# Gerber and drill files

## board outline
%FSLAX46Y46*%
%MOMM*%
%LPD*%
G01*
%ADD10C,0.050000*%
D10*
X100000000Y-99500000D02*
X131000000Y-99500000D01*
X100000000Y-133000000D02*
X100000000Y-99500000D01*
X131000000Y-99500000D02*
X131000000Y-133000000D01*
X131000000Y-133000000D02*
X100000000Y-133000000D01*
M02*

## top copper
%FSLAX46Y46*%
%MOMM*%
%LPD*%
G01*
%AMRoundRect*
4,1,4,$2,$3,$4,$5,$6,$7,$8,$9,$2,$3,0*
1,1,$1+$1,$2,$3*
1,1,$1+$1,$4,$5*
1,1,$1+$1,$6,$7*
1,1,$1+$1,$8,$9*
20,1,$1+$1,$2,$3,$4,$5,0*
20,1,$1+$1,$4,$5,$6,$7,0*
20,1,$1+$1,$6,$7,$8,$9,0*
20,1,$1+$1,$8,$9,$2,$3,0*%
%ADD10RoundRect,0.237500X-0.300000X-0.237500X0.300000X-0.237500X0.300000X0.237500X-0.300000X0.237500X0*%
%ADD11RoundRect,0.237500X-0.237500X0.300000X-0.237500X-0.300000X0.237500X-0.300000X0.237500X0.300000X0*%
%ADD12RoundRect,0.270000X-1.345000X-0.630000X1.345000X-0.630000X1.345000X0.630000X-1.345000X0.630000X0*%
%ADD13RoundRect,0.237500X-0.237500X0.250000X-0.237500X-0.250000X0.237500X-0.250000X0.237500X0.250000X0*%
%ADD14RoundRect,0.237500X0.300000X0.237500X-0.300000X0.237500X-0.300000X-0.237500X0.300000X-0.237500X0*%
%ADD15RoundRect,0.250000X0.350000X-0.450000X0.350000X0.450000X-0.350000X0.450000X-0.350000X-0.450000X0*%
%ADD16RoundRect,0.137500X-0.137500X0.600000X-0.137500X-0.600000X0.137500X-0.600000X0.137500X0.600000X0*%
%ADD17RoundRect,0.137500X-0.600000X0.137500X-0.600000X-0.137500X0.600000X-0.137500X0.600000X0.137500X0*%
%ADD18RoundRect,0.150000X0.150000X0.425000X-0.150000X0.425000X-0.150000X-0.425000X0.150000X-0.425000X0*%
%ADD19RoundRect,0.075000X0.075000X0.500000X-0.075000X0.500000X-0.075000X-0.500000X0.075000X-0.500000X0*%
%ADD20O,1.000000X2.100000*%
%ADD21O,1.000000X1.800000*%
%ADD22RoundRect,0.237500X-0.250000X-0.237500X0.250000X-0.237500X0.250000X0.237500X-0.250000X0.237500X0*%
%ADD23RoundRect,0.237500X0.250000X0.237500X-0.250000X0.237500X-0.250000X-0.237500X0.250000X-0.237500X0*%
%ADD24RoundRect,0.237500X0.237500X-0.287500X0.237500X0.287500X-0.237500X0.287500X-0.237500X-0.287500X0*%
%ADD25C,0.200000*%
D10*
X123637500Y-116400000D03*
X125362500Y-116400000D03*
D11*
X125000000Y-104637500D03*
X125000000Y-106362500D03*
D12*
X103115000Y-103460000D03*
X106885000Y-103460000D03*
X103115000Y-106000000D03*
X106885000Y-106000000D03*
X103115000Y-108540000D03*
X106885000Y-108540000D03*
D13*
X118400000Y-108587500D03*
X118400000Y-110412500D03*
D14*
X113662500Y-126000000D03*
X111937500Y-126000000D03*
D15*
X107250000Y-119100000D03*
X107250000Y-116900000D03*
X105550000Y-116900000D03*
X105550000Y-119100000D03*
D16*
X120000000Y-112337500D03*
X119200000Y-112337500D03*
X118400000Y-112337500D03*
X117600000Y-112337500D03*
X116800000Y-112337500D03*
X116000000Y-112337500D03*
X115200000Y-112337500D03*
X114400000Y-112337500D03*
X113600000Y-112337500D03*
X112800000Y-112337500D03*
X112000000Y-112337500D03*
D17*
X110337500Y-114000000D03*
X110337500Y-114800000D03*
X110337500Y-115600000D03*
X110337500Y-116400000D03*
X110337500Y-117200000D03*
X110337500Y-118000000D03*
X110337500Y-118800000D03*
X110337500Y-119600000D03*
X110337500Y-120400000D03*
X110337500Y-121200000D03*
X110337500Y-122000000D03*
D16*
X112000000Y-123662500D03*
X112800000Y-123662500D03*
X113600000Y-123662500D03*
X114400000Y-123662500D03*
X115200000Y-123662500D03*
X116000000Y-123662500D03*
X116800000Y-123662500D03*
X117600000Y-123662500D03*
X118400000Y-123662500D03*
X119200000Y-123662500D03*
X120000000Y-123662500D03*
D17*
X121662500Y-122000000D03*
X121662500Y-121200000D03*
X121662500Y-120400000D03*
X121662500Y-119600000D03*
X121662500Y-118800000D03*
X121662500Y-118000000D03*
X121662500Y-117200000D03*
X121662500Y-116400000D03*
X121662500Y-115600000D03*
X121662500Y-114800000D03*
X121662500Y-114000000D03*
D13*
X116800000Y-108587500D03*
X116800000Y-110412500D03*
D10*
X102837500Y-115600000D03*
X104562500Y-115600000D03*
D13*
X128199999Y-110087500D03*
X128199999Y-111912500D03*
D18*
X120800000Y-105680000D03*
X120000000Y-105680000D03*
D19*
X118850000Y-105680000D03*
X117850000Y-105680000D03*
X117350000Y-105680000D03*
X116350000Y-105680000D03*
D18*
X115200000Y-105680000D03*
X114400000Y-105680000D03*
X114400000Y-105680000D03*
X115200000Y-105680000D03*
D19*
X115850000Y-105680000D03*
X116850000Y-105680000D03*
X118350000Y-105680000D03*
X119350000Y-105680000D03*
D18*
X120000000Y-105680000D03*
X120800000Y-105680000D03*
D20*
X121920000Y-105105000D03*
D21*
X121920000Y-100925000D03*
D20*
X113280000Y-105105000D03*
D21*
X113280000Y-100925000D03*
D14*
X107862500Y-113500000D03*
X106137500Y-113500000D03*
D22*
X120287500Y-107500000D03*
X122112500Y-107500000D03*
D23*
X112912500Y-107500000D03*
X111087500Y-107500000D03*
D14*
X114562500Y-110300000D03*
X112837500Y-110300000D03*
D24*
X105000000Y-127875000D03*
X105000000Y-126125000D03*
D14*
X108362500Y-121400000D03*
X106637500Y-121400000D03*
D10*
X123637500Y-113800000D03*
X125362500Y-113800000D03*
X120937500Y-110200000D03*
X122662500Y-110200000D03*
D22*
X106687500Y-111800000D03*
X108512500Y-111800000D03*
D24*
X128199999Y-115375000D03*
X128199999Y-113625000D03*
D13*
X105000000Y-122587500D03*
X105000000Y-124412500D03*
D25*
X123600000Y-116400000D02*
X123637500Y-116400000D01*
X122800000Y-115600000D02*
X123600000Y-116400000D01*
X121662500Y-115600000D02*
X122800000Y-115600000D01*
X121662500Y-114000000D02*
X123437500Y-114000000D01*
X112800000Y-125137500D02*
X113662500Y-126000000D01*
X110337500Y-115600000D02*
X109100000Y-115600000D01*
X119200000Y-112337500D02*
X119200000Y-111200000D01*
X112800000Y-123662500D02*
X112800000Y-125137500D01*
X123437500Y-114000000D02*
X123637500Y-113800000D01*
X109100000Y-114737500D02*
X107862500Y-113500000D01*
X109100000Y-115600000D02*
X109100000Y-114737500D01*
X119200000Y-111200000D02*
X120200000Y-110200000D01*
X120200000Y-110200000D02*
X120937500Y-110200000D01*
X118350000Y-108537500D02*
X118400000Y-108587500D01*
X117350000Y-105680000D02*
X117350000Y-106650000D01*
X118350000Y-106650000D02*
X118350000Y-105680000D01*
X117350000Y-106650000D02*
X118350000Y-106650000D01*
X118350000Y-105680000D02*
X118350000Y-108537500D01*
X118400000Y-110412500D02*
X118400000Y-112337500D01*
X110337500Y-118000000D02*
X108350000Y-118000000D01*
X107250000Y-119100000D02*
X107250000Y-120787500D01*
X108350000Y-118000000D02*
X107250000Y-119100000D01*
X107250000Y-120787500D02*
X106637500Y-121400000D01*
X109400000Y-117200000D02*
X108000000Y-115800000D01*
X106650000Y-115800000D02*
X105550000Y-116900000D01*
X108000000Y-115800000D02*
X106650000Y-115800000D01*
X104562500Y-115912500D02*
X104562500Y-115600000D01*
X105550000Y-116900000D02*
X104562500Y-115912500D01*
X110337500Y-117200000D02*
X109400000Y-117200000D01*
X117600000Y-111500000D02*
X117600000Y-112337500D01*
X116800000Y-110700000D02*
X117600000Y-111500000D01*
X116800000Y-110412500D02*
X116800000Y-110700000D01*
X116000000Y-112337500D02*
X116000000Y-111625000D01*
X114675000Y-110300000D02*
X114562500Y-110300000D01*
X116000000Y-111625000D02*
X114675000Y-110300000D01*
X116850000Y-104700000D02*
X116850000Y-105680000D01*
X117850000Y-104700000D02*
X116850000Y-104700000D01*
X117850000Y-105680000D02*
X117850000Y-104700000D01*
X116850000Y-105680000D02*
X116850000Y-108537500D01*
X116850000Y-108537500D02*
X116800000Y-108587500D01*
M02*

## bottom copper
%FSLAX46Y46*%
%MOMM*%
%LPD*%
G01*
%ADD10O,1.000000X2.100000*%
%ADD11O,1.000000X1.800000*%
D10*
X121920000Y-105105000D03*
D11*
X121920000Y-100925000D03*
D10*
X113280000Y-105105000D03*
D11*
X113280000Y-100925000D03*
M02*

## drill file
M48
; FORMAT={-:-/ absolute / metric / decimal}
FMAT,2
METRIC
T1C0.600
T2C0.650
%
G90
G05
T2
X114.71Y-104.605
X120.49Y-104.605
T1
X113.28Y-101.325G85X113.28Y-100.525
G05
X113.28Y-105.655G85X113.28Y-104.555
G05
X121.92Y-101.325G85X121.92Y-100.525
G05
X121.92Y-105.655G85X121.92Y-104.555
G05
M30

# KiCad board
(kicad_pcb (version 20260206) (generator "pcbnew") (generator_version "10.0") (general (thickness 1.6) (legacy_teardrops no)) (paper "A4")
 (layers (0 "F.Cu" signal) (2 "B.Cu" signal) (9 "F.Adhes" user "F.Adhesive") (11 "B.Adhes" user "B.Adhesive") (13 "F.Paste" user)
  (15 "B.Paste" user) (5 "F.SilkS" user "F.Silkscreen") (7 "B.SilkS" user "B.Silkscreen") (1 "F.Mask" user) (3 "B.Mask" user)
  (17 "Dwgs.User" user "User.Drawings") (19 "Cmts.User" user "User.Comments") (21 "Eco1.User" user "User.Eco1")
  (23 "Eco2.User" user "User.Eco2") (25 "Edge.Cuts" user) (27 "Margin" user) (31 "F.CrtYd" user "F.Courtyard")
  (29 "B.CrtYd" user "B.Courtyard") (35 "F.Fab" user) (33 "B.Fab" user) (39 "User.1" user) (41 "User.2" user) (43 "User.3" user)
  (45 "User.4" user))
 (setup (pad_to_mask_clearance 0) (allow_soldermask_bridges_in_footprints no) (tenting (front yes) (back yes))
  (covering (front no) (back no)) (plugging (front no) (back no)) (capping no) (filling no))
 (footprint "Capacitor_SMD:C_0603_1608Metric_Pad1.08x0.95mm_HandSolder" (layer "F.Cu") (at 124.5 116.4)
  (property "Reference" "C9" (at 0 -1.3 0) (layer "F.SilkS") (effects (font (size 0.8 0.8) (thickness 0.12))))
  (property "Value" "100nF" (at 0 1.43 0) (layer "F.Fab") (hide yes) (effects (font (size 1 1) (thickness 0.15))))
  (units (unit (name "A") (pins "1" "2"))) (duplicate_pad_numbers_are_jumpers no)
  (pad "1" smd roundrect (at -0.8625 0) (size 1.075 0.95) (layers "F.Cu" "F.Mask" "F.Paste") (roundrect_rratio 0.25) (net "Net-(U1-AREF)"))
  (pad "2" smd roundrect (at 0.8625 0) (size 1.075 0.95) (layers "F.Cu" "F.Mask" "F.Paste") (roundrect_rratio 0.25) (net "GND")))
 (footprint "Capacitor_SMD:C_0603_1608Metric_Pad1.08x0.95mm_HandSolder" (layer "F.Cu") (at 125 105.5 -90)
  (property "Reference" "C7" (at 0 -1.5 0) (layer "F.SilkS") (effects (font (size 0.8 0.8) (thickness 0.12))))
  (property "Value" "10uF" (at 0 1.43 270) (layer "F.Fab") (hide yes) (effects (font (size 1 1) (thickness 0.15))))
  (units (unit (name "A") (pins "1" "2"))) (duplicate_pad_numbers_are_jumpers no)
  (pad "1" smd roundrect (at -0.8625 0 270) (size 1.075 0.95) (layers "F.Cu" "F.Mask" "F.Paste") (roundrect_rratio 0.25) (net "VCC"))
  (pad "2" smd roundrect (at 0.8625 0 270) (size 1.075 0.95) (layers "F.Cu" "F.Mask" "F.Paste") (roundrect_rratio 0.25) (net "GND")))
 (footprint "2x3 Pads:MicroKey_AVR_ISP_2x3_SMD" (layer "F.Cu") (at 105 106)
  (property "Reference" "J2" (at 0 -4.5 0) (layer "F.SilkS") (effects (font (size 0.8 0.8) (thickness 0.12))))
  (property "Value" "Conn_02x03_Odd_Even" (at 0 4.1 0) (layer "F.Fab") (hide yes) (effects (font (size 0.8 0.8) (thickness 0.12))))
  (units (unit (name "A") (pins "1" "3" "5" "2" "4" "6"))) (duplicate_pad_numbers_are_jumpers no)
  (pad "1" smd roundrect (at -1.885 -2.54) (size 3.23 1.8) (layers "F.Cu" "F.Mask" "F.Paste") (roundrect_rratio 0.15) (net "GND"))
  (pad "2" smd roundrect (at 1.885 -2.54) (size 3.23 1.8) (layers "F.Cu" "F.Mask" "F.Paste") (roundrect_rratio 0.15) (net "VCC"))
  (pad "3" smd roundrect (at -1.885 0) (size 3.23 1.8) (layers "F.Cu" "F.Mask" "F.Paste") (roundrect_rratio 0.15) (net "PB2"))
  (pad "4" smd roundrect (at 1.885 0) (size 3.23 1.8) (layers "F.Cu" "F.Mask" "F.Paste") (roundrect_rratio 0.15) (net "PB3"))
  (pad "5" smd roundrect (at -1.885 2.54) (size 3.23 1.8) (layers "F.Cu" "F.Mask" "F.Paste") (roundrect_rratio 0.15) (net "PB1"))
  (pad "6" smd roundrect (at 1.885 2.54) (size 3.23 1.8) (layers "F.Cu" "F.Mask" "F.Paste") (roundrect_rratio 0.15) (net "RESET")))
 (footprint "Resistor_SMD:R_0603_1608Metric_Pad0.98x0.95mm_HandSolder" (layer "F.Cu") (at 118.4 109.5 -90)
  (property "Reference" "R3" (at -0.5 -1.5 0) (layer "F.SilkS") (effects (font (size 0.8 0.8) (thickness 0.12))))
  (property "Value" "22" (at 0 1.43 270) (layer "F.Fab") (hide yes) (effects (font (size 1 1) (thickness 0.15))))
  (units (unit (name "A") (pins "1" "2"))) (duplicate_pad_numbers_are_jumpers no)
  (pad "1" smd roundrect (at -0.9125 0 270) (size 0.975 0.95) (layers "F.Cu" "F.Mask" "F.Paste") (roundrect_rratio 0.25)
   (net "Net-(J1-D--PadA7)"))
  (pad "2" smd roundrect (at 0.9125 0 270) (size 0.975 0.95) (layers "F.Cu" "F.Mask" "F.Paste") (roundrect_rratio 0.25) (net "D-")))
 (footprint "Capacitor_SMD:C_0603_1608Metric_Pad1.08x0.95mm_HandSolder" (layer "F.Cu") (at 112.8 126 180)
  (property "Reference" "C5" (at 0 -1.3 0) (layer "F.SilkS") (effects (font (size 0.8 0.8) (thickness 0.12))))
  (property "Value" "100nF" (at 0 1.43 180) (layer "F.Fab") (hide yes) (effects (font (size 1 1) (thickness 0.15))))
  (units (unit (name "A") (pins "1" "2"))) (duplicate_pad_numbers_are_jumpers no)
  (pad "1" smd roundrect (at -0.8625 0 180) (size 1.075 0.95) (layers "F.Cu" "F.Mask" "F.Paste") (roundrect_rratio 0.25) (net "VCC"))
  (pad "2" smd roundrect (at 0.8625 0 180) (size 1.075 0.95) (layers "F.Cu" "F.Mask" "F.Paste") (roundrect_rratio 0.25) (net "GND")))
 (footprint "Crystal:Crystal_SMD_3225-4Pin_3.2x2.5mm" (layer "F.Cu") (at 106.4 118 90)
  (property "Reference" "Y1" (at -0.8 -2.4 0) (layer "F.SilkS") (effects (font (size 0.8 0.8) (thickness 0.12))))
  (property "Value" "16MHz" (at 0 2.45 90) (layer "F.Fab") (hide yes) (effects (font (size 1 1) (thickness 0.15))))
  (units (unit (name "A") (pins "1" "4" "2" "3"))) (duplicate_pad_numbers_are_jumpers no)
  (pad "1" smd roundrect (at -1.1 0.85 90) (size 1.4 1.2) (layers "F.Cu" "F.Mask" "F.Paste") (roundrect_rratio 0.208333)
   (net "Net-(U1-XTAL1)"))
  (pad "2" smd roundrect (at 1.1 0.85 90) (size 1.4 1.2) (layers "F.Cu" "F.Mask" "F.Paste") (roundrect_rratio 0.208333) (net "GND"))
  (pad "3" smd roundrect (at 1.1 -0.85 90) (size 1.4 1.2) (layers "F.Cu" "F.Mask" "F.Paste") (roundrect_rratio 0.208333)
   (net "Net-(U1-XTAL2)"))
  (pad "4" smd roundrect (at -1.1 -0.85 90) (size 1.4 1.2) (layers "F.Cu" "F.Mask" "F.Paste") (roundrect_rratio 0.208333) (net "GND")))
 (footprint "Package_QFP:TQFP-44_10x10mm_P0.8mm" (layer "F.Cu") (at 116 118 -90)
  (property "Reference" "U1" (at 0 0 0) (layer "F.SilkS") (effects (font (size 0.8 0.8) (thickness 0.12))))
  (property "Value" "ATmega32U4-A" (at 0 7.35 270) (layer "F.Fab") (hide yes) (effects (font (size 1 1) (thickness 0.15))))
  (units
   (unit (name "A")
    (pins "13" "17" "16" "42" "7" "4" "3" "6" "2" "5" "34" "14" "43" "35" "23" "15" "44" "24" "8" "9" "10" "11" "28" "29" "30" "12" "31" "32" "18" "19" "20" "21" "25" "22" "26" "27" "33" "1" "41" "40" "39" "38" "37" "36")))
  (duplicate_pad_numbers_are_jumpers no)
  (pad "1" smd roundrect (at -5.6625 -4 270) (size 1.475 0.55) (layers "F.Cu" "F.Mask" "F.Paste") (roundrect_rratio 0.25)
   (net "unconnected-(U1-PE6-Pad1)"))
  (pad "2" smd roundrect (at -5.6625 -3.2 270) (size 1.475 0.55) (layers "F.Cu" "F.Mask" "F.Paste") (roundrect_rratio 0.25) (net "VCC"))
  (pad "3" smd roundrect (at -5.6625 -2.4 270) (size 1.475 0.55) (layers "F.Cu" "F.Mask" "F.Paste") (roundrect_rratio 0.25) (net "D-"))
  (pad "4" smd roundrect (at -5.6625 -1.6 270) (size 1.475 0.55) (layers "F.Cu" "F.Mask" "F.Paste") (roundrect_rratio 0.25) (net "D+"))
  (pad "5" smd roundrect (at -5.6625 -0.8 270) (size 1.475 0.55) (layers "F.Cu" "F.Mask" "F.Paste") (roundrect_rratio 0.25) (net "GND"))
  (pad "6" smd roundrect (at -5.6625 0 270) (size 1.475 0.55) (layers "F.Cu" "F.Mask" "F.Paste") (roundrect_rratio 0.25)
   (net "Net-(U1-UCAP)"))
  (pad "7" smd roundrect (at -5.6625 0.8 270) (size 1.475 0.55) (layers "F.Cu" "F.Mask" "F.Paste") (roundrect_rratio 0.25) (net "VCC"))
  (pad "8" smd roundrect (at -5.6625 1.6 270) (size 1.475 0.55) (layers "F.Cu" "F.Mask" "F.Paste") (roundrect_rratio 0.25)
   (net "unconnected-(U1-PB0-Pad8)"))
  (pad "9" smd roundrect (at -5.6625 2.4 270) (size 1.475 0.55) (layers "F.Cu" "F.Mask" "F.Paste") (roundrect_rratio 0.25) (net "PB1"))
  (pad "10" smd roundrect (at -5.6625 3.2 270) (size 1.475 0.55) (layers "F.Cu" "F.Mask" "F.Paste") (roundrect_rratio 0.25) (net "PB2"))
  (pad "11" smd roundrect (at -5.6625 4 270) (size 1.475 0.55) (layers "F.Cu" "F.Mask" "F.Paste") (roundrect_rratio 0.25) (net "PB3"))
  (pad "12" smd roundrect (at -4 5.6625 270) (size 0.55 1.475) (layers "F.Cu" "F.Mask" "F.Paste") (roundrect_rratio 0.25)
   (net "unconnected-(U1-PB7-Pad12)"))
  (pad "13" smd roundrect (at -3.2 5.6625 270) (size 0.55 1.475) (layers "F.Cu" "F.Mask" "F.Paste") (roundrect_rratio 0.25) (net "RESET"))
  (pad "14" smd roundrect (at -2.4 5.6625 270) (size 0.55 1.475) (layers "F.Cu" "F.Mask" "F.Paste") (roundrect_rratio 0.25) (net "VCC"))
  (pad "15" smd roundrect (at -1.6 5.6625 270) (size 0.55 1.475) (layers "F.Cu" "F.Mask" "F.Paste") (roundrect_rratio 0.25) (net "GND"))
  (pad "16" smd roundrect (at -0.8 5.6625 270) (size 0.55 1.475) (layers "F.Cu" "F.Mask" "F.Paste") (roundrect_rratio 0.25)
   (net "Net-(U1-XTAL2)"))
  (pad "17" smd roundrect (at 0 5.6625 270) (size 0.55 1.475) (layers "F.Cu" "F.Mask" "F.Paste") (roundrect_rratio 0.25)
   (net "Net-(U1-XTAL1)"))
  (pad "18" smd roundrect (at 0.8 5.6625 270) (size 0.55 1.475) (layers "F.Cu" "F.Mask" "F.Paste") (roundrect_rratio 0.25)
   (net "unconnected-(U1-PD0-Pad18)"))
  (pad "19" smd roundrect (at 1.6 5.6625 270) (size 0.55 1.475) (layers "F.Cu" "F.Mask" "F.Paste") (roundrect_rratio 0.25)
   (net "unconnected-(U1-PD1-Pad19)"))
  (pad "20" smd roundrect (at 2.4 5.6625 270) (size 0.55 1.475) (layers "F.Cu" "F.Mask" "F.Paste") (roundrect_rratio 0.25)
   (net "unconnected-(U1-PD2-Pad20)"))
  (pad "21" smd roundrect (at 3.2 5.6625 270) (size 0.55 1.475) (layers "F.Cu" "F.Mask" "F.Paste") (roundrect_rratio 0.25)
   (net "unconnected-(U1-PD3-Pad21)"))
  (pad "22" smd roundrect (at 4 5.6625 270) (size 0.55 1.475) (layers "F.Cu" "F.Mask" "F.Paste") (roundrect_rratio 0.25)
   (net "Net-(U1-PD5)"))
  (pad "23" smd roundrect (at 5.6625 4 270) (size 1.475 0.55) (layers "F.Cu" "F.Mask" "F.Paste") (roundrect_rratio 0.25) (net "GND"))
  (pad "24" smd roundrect (at 5.6625 3.2 270) (size 1.475 0.55) (layers "F.Cu" "F.Mask" "F.Paste") (roundrect_rratio 0.25) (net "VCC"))
  (pad "25" smd roundrect (at 5.6625 2.4 270) (size 1.475 0.55) (layers "F.Cu" "F.Mask" "F.Paste") (roundrect_rratio 0.25)
   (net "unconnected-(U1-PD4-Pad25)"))
  (pad "26" smd roundrect (at 5.6625 1.6 270) (size 1.475 0.55) (layers "F.Cu" "F.Mask" "F.Paste") (roundrect_rratio 0.25)
   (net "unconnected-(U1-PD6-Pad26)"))
  (pad "27" smd roundrect (at 5.6625 0.8 270) (size 1.475 0.55) (layers "F.Cu" "F.Mask" "F.Paste") (roundrect_rratio 0.25)
   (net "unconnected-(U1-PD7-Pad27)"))
  (pad "28" smd roundrect (at 5.6625 0 270) (size 1.475 0.55) (layers "F.Cu" "F.Mask" "F.Paste") (roundrect_rratio 0.25)
   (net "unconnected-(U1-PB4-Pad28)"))
  (pad "29" smd roundrect (at 5.6625 -0.8 270) (size 1.475 0.55) (layers "F.Cu" "F.Mask" "F.Paste") (roundrect_rratio 0.25)
   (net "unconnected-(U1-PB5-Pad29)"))
  (pad "30" smd roundrect (at 5.6625 -1.6 270) (size 1.475 0.55) (layers "F.Cu" "F.Mask" "F.Paste") (roundrect_rratio 0.25)
   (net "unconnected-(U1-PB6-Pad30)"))
  (pad "31" smd roundrect (at 5.6625 -2.4 270) (size 1.475 0.55) (layers "F.Cu" "F.Mask" "F.Paste") (roundrect_rratio 0.25)
   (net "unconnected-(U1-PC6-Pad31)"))
  (pad "32" smd roundrect (at 5.6625 -3.2 270) (size 1.475 0.55) (layers "F.Cu" "F.Mask" "F.Paste") (roundrect_rratio 0.25)
   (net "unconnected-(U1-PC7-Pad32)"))
  (pad "33" smd roundrect (at 5.6625 -4 270) (size 1.475 0.55) (layers "F.Cu" "F.Mask" "F.Paste") (roundrect_rratio 0.25)
   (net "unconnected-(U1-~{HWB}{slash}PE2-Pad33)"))
  (pad "34" smd roundrect (at 4 -5.6625 270) (size 0.55 1.475) (layers "F.Cu" "F.Mask" "F.Paste") (roundrect_rratio 0.25) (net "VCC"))
  (pad "35" smd roundrect (at 3.2 -5.6625 270) (size 0.55 1.475) (layers "F.Cu" "F.Mask" "F.Paste") (roundrect_rratio 0.25) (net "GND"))
  (pad "36" smd roundrect (at 2.4 -5.6625 270) (size 0.55 1.475) (layers "F.Cu" "F.Mask" "F.Paste") (roundrect_rratio 0.25)
   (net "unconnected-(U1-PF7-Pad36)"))
  (pad "37" smd roundrect (at 1.6 -5.6625 270) (size 0.55 1.475) (layers "F.Cu" "F.Mask" "F.Paste") (roundrect_rratio 0.25)
   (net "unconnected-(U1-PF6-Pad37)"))
  (pad "38" smd roundrect (at 0.8 -5.6625 270) (size 0.55 1.475) (layers "F.Cu" "F.Mask" "F.Paste") (roundrect_rratio 0.25)
   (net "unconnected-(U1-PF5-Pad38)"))
  (pad "39" smd roundrect (at 0 -5.6625 270) (size 0.55 1.475) (layers "F.Cu" "F.Mask" "F.Paste") (roundrect_rratio 0.25)
   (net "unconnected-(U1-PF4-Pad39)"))
  (pad "40" smd roundrect (at -0.8 -5.6625 270) (size 0.55 1.475) (layers "F.Cu" "F.Mask" "F.Paste") (roundrect_rratio 0.25)
   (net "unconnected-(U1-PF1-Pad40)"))
  (pad "41" smd roundrect (at -1.6 -5.6625 270) (size 0.55 1.475) (layers "F.Cu" "F.Mask" "F.Paste") (roundrect_rratio 0.25)
   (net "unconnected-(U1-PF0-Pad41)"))
  (pad "42" smd roundrect (at -2.4 -5.6625 270) (size 0.55 1.475) (layers "F.Cu" "F.Mask" "F.Paste") (roundrect_rratio 0.25)
   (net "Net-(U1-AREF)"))
  (pad "43" smd roundrect (at -3.2 -5.6625 270) (size 0.55 1.475) (layers "F.Cu" "F.Mask" "F.Paste") (roundrect_rratio 0.25) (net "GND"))
  (pad "44" smd roundrect (at -4 -5.6625 270) (size 0.55 1.475) (layers "F.Cu" "F.Mask" "F.Paste") (roundrect_rratio 0.25) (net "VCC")))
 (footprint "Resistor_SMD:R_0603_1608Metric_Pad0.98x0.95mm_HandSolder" (layer "F.Cu") (at 116.8 109.5 -90)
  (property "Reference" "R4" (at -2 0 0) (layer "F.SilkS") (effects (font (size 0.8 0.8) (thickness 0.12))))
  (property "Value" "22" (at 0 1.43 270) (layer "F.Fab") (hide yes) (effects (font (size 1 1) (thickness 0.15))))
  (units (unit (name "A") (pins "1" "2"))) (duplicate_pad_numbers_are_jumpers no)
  (pad "1" smd roundrect (at -0.9125 0 270) (size 0.975 0.95) (layers "F.Cu" "F.Mask" "F.Paste") (roundrect_rratio 0.25)
   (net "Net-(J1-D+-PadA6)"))
  (pad "2" smd roundrect (at 0.9125 0 270) (size 0.975 0.95) (layers "F.Cu" "F.Mask" "F.Paste") (roundrect_rratio 0.25) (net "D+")))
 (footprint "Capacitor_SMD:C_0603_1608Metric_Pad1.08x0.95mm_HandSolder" (layer "F.Cu") (at 103.7 115.6)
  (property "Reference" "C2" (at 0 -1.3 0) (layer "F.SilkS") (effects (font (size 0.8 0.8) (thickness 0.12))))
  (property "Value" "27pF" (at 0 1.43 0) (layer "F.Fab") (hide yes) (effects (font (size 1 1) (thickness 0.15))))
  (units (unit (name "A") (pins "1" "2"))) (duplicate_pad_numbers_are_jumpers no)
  (pad "1" smd roundrect (at -0.8625 0) (size 1.075 0.95) (layers "F.Cu" "F.Mask" "F.Paste") (roundrect_rratio 0.25) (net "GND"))
  (pad "2" smd roundrect (at 0.8625 0) (size 1.075 0.95) (layers "F.Cu" "F.Mask" "F.Paste") (roundrect_rratio 0.25) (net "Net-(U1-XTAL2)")))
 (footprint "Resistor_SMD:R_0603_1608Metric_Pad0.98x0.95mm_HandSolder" (layer "F.Cu") (at 128.199999 111 -90)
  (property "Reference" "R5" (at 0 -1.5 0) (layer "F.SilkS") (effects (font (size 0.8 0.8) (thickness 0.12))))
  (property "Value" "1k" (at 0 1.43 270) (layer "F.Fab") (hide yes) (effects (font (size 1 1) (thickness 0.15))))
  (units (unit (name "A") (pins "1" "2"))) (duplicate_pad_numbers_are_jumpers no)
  (pad "1" smd roundrect (at -0.9125 0 270) (size 0.975 0.95) (layers "F.Cu" "F.Mask" "F.Paste") (roundrect_rratio 0.25) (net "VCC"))
  (pad "2" smd roundrect (at 0.9125 0 270) (size 0.975 0.95) (layers "F.Cu" "F.Mask" "F.Paste") (roundrect_rratio 0.25) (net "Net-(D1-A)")))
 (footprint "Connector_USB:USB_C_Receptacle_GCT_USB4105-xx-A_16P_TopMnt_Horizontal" (layer "F.Cu") (at 117.6 102 180)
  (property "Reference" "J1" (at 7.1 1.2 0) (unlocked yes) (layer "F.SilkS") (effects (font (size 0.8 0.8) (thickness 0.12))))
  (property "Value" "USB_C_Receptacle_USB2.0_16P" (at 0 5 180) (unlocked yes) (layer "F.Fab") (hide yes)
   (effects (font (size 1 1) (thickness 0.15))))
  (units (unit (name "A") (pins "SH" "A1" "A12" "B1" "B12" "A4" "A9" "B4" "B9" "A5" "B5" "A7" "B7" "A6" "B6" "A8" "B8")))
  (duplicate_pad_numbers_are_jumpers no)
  (pad "" np_thru_hole circle (at -2.89 -2.605 180) (size 0.65 0.65) (drill 0.65) (layers "*.Cu" "*.Mask"))
  (pad "" np_thru_hole circle (at 2.89 -2.605 180) (size 0.65 0.65) (drill 0.65) (layers "*.Cu" "*.Mask"))
  (pad "A1" smd roundrect (at -3.2 -3.68 180) (size 0.6 1.15) (layers "F.Cu" "F.Mask" "F.Paste") (roundrect_rratio 0.25) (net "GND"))
  (pad "A4" smd roundrect (at -2.4 -3.68 180) (size 0.6 1.15) (layers "F.Cu" "F.Mask" "F.Paste") (roundrect_rratio 0.25) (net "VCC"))
  (pad "A5" smd roundrect (at -1.25 -3.68 180) (size 0.3 1.15) (layers "F.Cu" "F.Mask" "F.Paste") (roundrect_rratio 0.25)
   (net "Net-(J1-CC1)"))
  (pad "A6" smd roundrect (at -0.25 -3.68 180) (size 0.3 1.15) (layers "F.Cu" "F.Mask" "F.Paste") (roundrect_rratio 0.25)
   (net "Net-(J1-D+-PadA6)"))
  (pad "A7" smd roundrect (at 0.25 -3.68 180) (size 0.3 1.15) (layers "F.Cu" "F.Mask" "F.Paste") (roundrect_rratio 0.25)
   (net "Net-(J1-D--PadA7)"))
  (pad "A8" smd roundrect (at 1.25 -3.68 180) (size 0.3 1.15) (layers "F.Cu" "F.Mask" "F.Paste") (roundrect_rratio 0.25)
   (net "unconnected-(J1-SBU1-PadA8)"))
  (pad "A9" smd roundrect (at 2.4 -3.68 180) (size 0.6 1.15) (layers "F.Cu" "F.Mask" "F.Paste") (roundrect_rratio 0.25) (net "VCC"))
  (pad "A12" smd roundrect (at 3.2 -3.68 180) (size 0.6 1.15) (layers "F.Cu" "F.Mask" "F.Paste") (roundrect_rratio 0.25) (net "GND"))
  (pad "B1" smd roundrect (at 3.2 -3.68 180) (size 0.6 1.15) (layers "F.Cu" "F.Mask" "F.Paste") (roundrect_rratio 0.25) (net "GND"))
  (pad "B4" smd roundrect (at 2.4 -3.68 180) (size 0.6 1.15) (layers "F.Cu" "F.Mask" "F.Paste") (roundrect_rratio 0.25) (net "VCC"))
  (pad "B5" smd roundrect (at 1.75 -3.68 180) (size 0.3 1.15) (layers "F.Cu" "F.Mask" "F.Paste") (roundrect_rratio 0.25)
   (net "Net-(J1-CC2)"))
  (pad "B6" smd roundrect (at 0.75 -3.68 180) (size 0.3 1.15) (layers "F.Cu" "F.Mask" "F.Paste") (roundrect_rratio 0.25)
   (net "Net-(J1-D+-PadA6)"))
  (pad "B7" smd roundrect (at -0.75 -3.68 180) (size 0.3 1.15) (layers "F.Cu" "F.Mask" "F.Paste") (roundrect_rratio 0.25)
   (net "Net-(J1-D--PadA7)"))
  (pad "B8" smd roundrect (at -1.75 -3.68 180) (size 0.3 1.15) (layers "F.Cu" "F.Mask" "F.Paste") (roundrect_rratio 0.25)
   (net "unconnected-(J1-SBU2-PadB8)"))
  (pad "B9" smd roundrect (at -2.4 -3.68 180) (size 0.6 1.15) (layers "F.Cu" "F.Mask" "F.Paste") (roundrect_rratio 0.25) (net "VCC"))
  (pad "B12" smd roundrect (at -3.2 -3.68 180) (size 0.6 1.15) (layers "F.Cu" "F.Mask" "F.Paste") (roundrect_rratio 0.25) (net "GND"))
  (pad "SH" thru_hole oval (at -4.32 -3.105 180) (size 1 2.1) (drill oval 0.6 1.7) (layers "*.Cu" "*.Mask" "F.Paste")
   (remove_unused_layers no) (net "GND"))
  (pad "SH" thru_hole oval (at -4.32 1.075 180) (size 1 1.8) (drill oval 0.6 1.4) (layers "*.Cu" "*.Mask" "F.Paste")
   (remove_unused_layers no) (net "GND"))
  (pad "SH" thru_hole oval (at 4.32 -3.105 180) (size 1 2.1) (drill oval 0.6 1.7) (layers "*.Cu" "*.Mask" "F.Paste")
   (remove_unused_layers no) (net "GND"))
  (pad "SH" thru_hole oval (at 4.32 1.075 180) (size 1 1.8) (drill oval 0.6 1.4) (layers "*.Cu" "*.Mask" "F.Paste")
   (remove_unused_layers no) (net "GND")))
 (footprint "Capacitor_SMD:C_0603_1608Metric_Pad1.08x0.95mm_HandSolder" (layer "F.Cu") (at 107 113.5 180)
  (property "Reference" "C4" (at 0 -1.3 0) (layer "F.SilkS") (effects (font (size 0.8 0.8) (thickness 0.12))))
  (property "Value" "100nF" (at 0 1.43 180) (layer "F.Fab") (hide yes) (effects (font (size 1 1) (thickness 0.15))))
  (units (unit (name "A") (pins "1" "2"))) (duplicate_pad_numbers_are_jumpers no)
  (pad "1" smd roundrect (at -0.8625 0 180) (size 1.075 0.95) (layers "F.Cu" "F.Mask" "F.Paste") (roundrect_rratio 0.25) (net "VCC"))
  (pad "2" smd roundrect (at 0.8625 0 180) (size 1.075 0.95) (layers "F.Cu" "F.Mask" "F.Paste") (roundrect_rratio 0.25) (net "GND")))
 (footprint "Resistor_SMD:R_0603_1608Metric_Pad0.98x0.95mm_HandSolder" (layer "F.Cu") (at 121.2 107.5)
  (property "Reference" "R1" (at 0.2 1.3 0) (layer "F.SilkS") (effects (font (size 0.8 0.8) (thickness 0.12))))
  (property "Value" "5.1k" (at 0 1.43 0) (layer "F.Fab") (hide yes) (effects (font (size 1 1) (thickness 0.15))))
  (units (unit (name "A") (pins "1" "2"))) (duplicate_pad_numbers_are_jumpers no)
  (pad "1" smd roundrect (at -0.9125 0) (size 0.975 0.95) (layers "F.Cu" "F.Mask" "F.Paste") (roundrect_rratio 0.25) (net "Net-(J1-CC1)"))
  (pad "2" smd roundrect (at 0.9125 0) (size 0.975 0.95) (layers "F.Cu" "F.Mask" "F.Paste") (roundrect_rratio 0.25) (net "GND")))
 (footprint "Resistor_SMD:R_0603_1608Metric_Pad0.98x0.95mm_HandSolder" (layer "F.Cu") (at 112 107.5 180)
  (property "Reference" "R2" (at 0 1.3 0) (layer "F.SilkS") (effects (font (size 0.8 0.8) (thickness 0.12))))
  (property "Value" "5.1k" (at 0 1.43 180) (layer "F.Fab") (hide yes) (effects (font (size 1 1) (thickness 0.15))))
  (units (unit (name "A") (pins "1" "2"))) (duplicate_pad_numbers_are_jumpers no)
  (pad "1" smd roundrect (at -0.9125 0 180) (size 0.975 0.95) (layers "F.Cu" "F.Mask" "F.Paste") (roundrect_rratio 0.25)
   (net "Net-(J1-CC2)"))
  (pad "2" smd roundrect (at 0.9125 0 180) (size 0.975 0.95) (layers "F.Cu" "F.Mask" "F.Paste") (roundrect_rratio 0.25) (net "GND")))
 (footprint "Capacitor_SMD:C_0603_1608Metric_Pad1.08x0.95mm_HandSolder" (layer "F.Cu") (at 113.7 110.3 180)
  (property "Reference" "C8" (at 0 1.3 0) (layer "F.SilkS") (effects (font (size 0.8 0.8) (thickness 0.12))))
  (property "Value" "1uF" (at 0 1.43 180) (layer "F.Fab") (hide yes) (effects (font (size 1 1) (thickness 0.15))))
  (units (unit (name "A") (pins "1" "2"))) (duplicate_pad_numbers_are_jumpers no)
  (pad "1" smd roundrect (at -0.8625 0 180) (size 1.075 0.95) (layers "F.Cu" "F.Mask" "F.Paste") (roundrect_rratio 0.25)
   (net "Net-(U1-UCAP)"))
  (pad "2" smd roundrect (at 0.8625 0 180) (size 1.075 0.95) (layers "F.Cu" "F.Mask" "F.Paste") (roundrect_rratio 0.25) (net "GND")))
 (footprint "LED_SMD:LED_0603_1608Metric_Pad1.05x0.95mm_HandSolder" (layer "F.Cu") (at 105 127 90)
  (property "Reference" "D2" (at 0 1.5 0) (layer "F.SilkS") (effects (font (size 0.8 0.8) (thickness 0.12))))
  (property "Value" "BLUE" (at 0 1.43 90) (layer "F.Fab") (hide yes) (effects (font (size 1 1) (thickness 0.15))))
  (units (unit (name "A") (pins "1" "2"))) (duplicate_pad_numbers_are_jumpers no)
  (pad "1" smd roundrect (at -0.875 0 90) (size 1.05 0.95) (layers "F.Cu" "F.Mask" "F.Paste") (roundrect_rratio 0.25) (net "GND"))
  (pad "2" smd roundrect (at 0.875 0 90) (size 1.05 0.95) (layers "F.Cu" "F.Mask" "F.Paste") (roundrect_rratio 0.25) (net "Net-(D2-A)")))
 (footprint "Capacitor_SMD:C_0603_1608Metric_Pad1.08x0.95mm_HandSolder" (layer "F.Cu") (at 107.5 121.4 180)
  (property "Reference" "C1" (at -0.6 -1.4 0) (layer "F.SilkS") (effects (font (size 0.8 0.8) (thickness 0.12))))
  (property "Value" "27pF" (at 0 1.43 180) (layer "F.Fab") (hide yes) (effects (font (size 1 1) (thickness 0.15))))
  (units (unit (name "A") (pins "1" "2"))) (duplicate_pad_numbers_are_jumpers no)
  (pad "1" smd roundrect (at -0.8625 0 180) (size 1.075 0.95) (layers "F.Cu" "F.Mask" "F.Paste") (roundrect_rratio 0.25) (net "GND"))
  (pad "2" smd roundrect (at 0.8625 0 180) (size 1.075 0.95) (layers "F.Cu" "F.Mask" "F.Paste") (roundrect_rratio 0.25)
   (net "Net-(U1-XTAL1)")))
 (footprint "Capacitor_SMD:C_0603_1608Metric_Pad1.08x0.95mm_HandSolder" (layer "F.Cu") (at 124.5 113.8)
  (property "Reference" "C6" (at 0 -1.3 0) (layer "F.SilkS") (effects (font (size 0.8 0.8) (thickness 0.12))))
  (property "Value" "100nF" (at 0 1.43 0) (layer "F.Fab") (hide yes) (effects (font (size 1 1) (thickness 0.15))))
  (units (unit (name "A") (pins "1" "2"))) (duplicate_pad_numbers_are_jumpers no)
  (pad "1" smd roundrect (at -0.8625 0) (size 1.075 0.95) (layers "F.Cu" "F.Mask" "F.Paste") (roundrect_rratio 0.25) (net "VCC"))
  (pad "2" smd roundrect (at 0.8625 0) (size 1.075 0.95) (layers "F.Cu" "F.Mask" "F.Paste") (roundrect_rratio 0.25) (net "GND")))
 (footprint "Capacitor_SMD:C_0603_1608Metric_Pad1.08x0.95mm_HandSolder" (layer "F.Cu") (at 121.8 110.2)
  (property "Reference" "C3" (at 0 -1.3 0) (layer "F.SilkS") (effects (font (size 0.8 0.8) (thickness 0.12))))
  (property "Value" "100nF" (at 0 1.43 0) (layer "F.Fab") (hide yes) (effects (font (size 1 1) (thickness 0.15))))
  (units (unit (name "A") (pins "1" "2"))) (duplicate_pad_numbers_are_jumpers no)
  (pad "1" smd roundrect (at -0.8625 0) (size 1.075 0.95) (layers "F.Cu" "F.Mask" "F.Paste") (roundrect_rratio 0.25) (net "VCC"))
  (pad "2" smd roundrect (at 0.8625 0) (size 1.075 0.95) (layers "F.Cu" "F.Mask" "F.Paste") (roundrect_rratio 0.25) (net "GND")))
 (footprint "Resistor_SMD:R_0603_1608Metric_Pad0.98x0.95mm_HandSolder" (layer "F.Cu") (at 107.6 111.8)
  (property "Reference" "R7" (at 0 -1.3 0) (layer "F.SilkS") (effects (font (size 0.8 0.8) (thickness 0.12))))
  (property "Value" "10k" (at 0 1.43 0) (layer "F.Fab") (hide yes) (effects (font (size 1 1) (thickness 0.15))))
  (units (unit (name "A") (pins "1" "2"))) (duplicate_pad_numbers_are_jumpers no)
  (pad "1" smd roundrect (at -0.9125 0) (size 0.975 0.95) (layers "F.Cu" "F.Mask" "F.Paste") (roundrect_rratio 0.25) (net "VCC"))
  (pad "2" smd roundrect (at 0.9125 0) (size 0.975 0.95) (layers "F.Cu" "F.Mask" "F.Paste") (roundrect_rratio 0.25) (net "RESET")))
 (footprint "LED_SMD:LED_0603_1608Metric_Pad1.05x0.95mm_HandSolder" (layer "F.Cu") (at 128.199999 114.5 90)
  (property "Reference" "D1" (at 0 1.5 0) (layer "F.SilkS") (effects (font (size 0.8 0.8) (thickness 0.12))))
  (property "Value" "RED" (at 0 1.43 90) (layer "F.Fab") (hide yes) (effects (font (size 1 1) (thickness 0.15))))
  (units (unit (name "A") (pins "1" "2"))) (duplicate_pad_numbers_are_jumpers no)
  (pad "1" smd roundrect (at -0.875 0 90) (size 1.05 0.95) (layers "F.Cu" "F.Mask" "F.Paste") (roundrect_rratio 0.25) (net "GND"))
  (pad "2" smd roundrect (at 0.875 0 90) (size 1.05 0.95) (layers "F.Cu" "F.Mask" "F.Paste") (roundrect_rratio 0.25) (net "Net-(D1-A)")))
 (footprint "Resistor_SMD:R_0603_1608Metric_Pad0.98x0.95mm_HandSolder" (layer "F.Cu") (at 105 123.5 -90)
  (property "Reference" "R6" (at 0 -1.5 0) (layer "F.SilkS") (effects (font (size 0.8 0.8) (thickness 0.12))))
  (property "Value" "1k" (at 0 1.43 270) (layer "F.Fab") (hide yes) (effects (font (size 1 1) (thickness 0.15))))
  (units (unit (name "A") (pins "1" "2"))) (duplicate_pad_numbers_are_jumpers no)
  (pad "1" smd roundrect (at -0.9125 0 270) (size 0.975 0.95) (layers "F.Cu" "F.Mask" "F.Paste") (roundrect_rratio 0.25)
   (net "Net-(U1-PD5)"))
  (pad "2" smd roundrect (at 0.9125 0 270) (size 0.975 0.95) (layers "F.Cu" "F.Mask" "F.Paste") (roundrect_rratio 0.25) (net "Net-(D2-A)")))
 (gr_line (start 100 99.5) (end 131 99.5) (stroke (width 0.05) (type default)) (layer "Edge.Cuts"))
 (gr_line (start 100 133) (end 100 99.5) (stroke (width 0.05) (type default)) (layer "Edge.Cuts"))
 (gr_line (start 131 99.5) (end 131 133) (stroke (width 0.05) (type default)) (layer "Edge.Cuts"))
 (gr_line (start 131 133) (end 100 133) (stroke (width 0.05) (type default)) (layer "Edge.Cuts"))
 (segment (start 123.6 116.4) (end 123.6375 116.4) (width 0.2) (locked yes) (layer "F.Cu") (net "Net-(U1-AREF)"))
 (segment (start 122.8 115.6) (end 123.6 116.4) (width 0.2) (locked yes) (layer "F.Cu") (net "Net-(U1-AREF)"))
 (segment (start 121.6625 115.6) (end 122.8 115.6) (width 0.2) (locked yes) (layer "F.Cu") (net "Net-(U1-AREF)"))
 (segment (start 121.6625 114) (end 123.4375 114) (width 0.2) (locked yes) (layer "F.Cu") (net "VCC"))
 (segment (start 112.8 125.1375) (end 113.6625 126) (width 0.2) (locked yes) (layer "F.Cu") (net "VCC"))
 (segment (start 110.3375 115.6) (end 109.1 115.6) (width 0.2) (locked yes) (layer "F.Cu") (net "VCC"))
 (segment (start 119.2 112.3375) (end 119.2 111.2) (width 0.2) (locked yes) (layer "F.Cu") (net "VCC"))
 (segment (start 112.8 123.6625) (end 112.8 125.1375) (width 0.2) (locked yes) (layer "F.Cu") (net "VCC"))
 (segment (start 123.4375 114) (end 123.6375 113.8) (width 0.2) (locked yes) (layer "F.Cu") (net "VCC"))
 (segment (start 109.1 114.7375) (end 107.8625 113.5) (width 0.2) (locked yes) (layer "F.Cu") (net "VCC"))
 (segment (start 109.1 115.6) (end 109.1 114.7375) (width 0.2) (locked yes) (layer "F.Cu") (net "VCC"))
 (segment (start 119.2 111.2) (end 120.2 110.2) (width 0.2) (locked yes) (layer "F.Cu") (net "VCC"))
 (segment (start 120.2 110.2) (end 120.9375 110.2) (width 0.2) (locked yes) (layer "F.Cu") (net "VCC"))
 (segment (start 118.35 108.5375) (end 118.4 108.5875) (width 0.2) (locked yes) (layer "F.Cu") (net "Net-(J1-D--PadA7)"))
 (segment (start 117.35 105.68) (end 117.35 106.65) (width 0.2) (locked yes) (layer "F.Cu") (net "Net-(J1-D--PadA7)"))
 (segment (start 118.35 106.65) (end 118.35 105.68) (width 0.2) (locked yes) (layer "F.Cu") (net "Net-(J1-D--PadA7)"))
 (segment (start 117.35 106.65) (end 118.35 106.65) (width 0.2) (locked yes) (layer "F.Cu") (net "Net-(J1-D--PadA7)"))
 (segment (start 118.35 105.68) (end 118.35 108.5375) (width 0.2) (locked yes) (layer "F.Cu") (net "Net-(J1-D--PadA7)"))
 (segment (start 118.4 110.4125) (end 118.4 112.3375) (width 0.2) (locked yes) (layer "F.Cu") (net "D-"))
 (segment (start 110.3375 118) (end 108.35 118) (width 0.2) (locked yes) (layer "F.Cu") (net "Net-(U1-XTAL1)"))
 (segment (start 107.25 119.1) (end 107.25 120.7875) (width 0.2) (locked yes) (layer "F.Cu") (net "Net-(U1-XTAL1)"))
 (segment (start 108.35 118) (end 107.25 119.1) (width 0.2) (locked yes) (layer "F.Cu") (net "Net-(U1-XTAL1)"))
 (segment (start 107.25 120.7875) (end 106.6375 121.4) (width 0.2) (locked yes) (layer "F.Cu") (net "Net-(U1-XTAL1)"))
 (segment (start 109.4 117.2) (end 108 115.8) (width 0.2) (locked yes) (layer "F.Cu") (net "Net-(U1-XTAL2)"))
 (segment (start 106.65 115.8) (end 105.55 116.9) (width 0.2) (locked yes) (layer "F.Cu") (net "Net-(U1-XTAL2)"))
 (segment (start 108 115.8) (end 106.65 115.8) (width 0.2) (locked yes) (layer "F.Cu") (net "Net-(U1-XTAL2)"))
 (segment (start 104.5625 115.9125) (end 104.5625 115.6) (width 0.2) (locked yes) (layer "F.Cu") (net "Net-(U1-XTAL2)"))
 (segment (start 105.55 116.9) (end 104.5625 115.9125) (width 0.2) (locked yes) (layer "F.Cu") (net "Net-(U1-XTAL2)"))
 (segment (start 110.3375 117.2) (end 109.4 117.2) (width 0.2) (locked yes) (layer "F.Cu") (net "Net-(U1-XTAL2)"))
 (segment (start 117.6 111.5) (end 117.6 112.3375) (width 0.2) (locked yes) (layer "F.Cu") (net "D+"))
 (segment (start 116.8 110.7) (end 117.6 111.5) (width 0.2) (locked yes) (layer "F.Cu") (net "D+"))
 (segment (start 116.8 110.4125) (end 116.8 110.7) (width 0.2) (locked yes) (layer "F.Cu") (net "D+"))
 (segment (start 116 112.3375) (end 116 111.625) (width 0.2) (locked yes) (layer "F.Cu") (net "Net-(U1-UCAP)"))
 (segment (start 114.675 110.3) (end 114.5625 110.3) (width 0.2) (locked yes) (layer "F.Cu") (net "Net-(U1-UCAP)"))
 (segment (start 116 111.625) (end 114.675 110.3) (width 0.2) (locked yes) (layer "F.Cu") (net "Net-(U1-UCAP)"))
 (segment (start 116.85 104.7) (end 116.85 105.68) (width 0.2) (locked yes) (layer "F.Cu") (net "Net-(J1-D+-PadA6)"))
 (segment (start 117.85 104.7) (end 116.85 104.7) (width 0.2) (locked yes) (layer "F.Cu") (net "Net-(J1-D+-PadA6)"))
 (segment (start 117.85 105.68) (end 117.85 104.7) (width 0.2) (locked yes) (layer "F.Cu") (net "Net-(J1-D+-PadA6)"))
 (segment (start 116.85 105.68) (end 116.85 108.5375) (width 0.2) (locked yes) (layer "F.Cu") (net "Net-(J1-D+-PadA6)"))
 (segment (start 116.85 108.5375) (end 116.8 108.5875) (width 0.2) (locked yes) (layer "F.Cu") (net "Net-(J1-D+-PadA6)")))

